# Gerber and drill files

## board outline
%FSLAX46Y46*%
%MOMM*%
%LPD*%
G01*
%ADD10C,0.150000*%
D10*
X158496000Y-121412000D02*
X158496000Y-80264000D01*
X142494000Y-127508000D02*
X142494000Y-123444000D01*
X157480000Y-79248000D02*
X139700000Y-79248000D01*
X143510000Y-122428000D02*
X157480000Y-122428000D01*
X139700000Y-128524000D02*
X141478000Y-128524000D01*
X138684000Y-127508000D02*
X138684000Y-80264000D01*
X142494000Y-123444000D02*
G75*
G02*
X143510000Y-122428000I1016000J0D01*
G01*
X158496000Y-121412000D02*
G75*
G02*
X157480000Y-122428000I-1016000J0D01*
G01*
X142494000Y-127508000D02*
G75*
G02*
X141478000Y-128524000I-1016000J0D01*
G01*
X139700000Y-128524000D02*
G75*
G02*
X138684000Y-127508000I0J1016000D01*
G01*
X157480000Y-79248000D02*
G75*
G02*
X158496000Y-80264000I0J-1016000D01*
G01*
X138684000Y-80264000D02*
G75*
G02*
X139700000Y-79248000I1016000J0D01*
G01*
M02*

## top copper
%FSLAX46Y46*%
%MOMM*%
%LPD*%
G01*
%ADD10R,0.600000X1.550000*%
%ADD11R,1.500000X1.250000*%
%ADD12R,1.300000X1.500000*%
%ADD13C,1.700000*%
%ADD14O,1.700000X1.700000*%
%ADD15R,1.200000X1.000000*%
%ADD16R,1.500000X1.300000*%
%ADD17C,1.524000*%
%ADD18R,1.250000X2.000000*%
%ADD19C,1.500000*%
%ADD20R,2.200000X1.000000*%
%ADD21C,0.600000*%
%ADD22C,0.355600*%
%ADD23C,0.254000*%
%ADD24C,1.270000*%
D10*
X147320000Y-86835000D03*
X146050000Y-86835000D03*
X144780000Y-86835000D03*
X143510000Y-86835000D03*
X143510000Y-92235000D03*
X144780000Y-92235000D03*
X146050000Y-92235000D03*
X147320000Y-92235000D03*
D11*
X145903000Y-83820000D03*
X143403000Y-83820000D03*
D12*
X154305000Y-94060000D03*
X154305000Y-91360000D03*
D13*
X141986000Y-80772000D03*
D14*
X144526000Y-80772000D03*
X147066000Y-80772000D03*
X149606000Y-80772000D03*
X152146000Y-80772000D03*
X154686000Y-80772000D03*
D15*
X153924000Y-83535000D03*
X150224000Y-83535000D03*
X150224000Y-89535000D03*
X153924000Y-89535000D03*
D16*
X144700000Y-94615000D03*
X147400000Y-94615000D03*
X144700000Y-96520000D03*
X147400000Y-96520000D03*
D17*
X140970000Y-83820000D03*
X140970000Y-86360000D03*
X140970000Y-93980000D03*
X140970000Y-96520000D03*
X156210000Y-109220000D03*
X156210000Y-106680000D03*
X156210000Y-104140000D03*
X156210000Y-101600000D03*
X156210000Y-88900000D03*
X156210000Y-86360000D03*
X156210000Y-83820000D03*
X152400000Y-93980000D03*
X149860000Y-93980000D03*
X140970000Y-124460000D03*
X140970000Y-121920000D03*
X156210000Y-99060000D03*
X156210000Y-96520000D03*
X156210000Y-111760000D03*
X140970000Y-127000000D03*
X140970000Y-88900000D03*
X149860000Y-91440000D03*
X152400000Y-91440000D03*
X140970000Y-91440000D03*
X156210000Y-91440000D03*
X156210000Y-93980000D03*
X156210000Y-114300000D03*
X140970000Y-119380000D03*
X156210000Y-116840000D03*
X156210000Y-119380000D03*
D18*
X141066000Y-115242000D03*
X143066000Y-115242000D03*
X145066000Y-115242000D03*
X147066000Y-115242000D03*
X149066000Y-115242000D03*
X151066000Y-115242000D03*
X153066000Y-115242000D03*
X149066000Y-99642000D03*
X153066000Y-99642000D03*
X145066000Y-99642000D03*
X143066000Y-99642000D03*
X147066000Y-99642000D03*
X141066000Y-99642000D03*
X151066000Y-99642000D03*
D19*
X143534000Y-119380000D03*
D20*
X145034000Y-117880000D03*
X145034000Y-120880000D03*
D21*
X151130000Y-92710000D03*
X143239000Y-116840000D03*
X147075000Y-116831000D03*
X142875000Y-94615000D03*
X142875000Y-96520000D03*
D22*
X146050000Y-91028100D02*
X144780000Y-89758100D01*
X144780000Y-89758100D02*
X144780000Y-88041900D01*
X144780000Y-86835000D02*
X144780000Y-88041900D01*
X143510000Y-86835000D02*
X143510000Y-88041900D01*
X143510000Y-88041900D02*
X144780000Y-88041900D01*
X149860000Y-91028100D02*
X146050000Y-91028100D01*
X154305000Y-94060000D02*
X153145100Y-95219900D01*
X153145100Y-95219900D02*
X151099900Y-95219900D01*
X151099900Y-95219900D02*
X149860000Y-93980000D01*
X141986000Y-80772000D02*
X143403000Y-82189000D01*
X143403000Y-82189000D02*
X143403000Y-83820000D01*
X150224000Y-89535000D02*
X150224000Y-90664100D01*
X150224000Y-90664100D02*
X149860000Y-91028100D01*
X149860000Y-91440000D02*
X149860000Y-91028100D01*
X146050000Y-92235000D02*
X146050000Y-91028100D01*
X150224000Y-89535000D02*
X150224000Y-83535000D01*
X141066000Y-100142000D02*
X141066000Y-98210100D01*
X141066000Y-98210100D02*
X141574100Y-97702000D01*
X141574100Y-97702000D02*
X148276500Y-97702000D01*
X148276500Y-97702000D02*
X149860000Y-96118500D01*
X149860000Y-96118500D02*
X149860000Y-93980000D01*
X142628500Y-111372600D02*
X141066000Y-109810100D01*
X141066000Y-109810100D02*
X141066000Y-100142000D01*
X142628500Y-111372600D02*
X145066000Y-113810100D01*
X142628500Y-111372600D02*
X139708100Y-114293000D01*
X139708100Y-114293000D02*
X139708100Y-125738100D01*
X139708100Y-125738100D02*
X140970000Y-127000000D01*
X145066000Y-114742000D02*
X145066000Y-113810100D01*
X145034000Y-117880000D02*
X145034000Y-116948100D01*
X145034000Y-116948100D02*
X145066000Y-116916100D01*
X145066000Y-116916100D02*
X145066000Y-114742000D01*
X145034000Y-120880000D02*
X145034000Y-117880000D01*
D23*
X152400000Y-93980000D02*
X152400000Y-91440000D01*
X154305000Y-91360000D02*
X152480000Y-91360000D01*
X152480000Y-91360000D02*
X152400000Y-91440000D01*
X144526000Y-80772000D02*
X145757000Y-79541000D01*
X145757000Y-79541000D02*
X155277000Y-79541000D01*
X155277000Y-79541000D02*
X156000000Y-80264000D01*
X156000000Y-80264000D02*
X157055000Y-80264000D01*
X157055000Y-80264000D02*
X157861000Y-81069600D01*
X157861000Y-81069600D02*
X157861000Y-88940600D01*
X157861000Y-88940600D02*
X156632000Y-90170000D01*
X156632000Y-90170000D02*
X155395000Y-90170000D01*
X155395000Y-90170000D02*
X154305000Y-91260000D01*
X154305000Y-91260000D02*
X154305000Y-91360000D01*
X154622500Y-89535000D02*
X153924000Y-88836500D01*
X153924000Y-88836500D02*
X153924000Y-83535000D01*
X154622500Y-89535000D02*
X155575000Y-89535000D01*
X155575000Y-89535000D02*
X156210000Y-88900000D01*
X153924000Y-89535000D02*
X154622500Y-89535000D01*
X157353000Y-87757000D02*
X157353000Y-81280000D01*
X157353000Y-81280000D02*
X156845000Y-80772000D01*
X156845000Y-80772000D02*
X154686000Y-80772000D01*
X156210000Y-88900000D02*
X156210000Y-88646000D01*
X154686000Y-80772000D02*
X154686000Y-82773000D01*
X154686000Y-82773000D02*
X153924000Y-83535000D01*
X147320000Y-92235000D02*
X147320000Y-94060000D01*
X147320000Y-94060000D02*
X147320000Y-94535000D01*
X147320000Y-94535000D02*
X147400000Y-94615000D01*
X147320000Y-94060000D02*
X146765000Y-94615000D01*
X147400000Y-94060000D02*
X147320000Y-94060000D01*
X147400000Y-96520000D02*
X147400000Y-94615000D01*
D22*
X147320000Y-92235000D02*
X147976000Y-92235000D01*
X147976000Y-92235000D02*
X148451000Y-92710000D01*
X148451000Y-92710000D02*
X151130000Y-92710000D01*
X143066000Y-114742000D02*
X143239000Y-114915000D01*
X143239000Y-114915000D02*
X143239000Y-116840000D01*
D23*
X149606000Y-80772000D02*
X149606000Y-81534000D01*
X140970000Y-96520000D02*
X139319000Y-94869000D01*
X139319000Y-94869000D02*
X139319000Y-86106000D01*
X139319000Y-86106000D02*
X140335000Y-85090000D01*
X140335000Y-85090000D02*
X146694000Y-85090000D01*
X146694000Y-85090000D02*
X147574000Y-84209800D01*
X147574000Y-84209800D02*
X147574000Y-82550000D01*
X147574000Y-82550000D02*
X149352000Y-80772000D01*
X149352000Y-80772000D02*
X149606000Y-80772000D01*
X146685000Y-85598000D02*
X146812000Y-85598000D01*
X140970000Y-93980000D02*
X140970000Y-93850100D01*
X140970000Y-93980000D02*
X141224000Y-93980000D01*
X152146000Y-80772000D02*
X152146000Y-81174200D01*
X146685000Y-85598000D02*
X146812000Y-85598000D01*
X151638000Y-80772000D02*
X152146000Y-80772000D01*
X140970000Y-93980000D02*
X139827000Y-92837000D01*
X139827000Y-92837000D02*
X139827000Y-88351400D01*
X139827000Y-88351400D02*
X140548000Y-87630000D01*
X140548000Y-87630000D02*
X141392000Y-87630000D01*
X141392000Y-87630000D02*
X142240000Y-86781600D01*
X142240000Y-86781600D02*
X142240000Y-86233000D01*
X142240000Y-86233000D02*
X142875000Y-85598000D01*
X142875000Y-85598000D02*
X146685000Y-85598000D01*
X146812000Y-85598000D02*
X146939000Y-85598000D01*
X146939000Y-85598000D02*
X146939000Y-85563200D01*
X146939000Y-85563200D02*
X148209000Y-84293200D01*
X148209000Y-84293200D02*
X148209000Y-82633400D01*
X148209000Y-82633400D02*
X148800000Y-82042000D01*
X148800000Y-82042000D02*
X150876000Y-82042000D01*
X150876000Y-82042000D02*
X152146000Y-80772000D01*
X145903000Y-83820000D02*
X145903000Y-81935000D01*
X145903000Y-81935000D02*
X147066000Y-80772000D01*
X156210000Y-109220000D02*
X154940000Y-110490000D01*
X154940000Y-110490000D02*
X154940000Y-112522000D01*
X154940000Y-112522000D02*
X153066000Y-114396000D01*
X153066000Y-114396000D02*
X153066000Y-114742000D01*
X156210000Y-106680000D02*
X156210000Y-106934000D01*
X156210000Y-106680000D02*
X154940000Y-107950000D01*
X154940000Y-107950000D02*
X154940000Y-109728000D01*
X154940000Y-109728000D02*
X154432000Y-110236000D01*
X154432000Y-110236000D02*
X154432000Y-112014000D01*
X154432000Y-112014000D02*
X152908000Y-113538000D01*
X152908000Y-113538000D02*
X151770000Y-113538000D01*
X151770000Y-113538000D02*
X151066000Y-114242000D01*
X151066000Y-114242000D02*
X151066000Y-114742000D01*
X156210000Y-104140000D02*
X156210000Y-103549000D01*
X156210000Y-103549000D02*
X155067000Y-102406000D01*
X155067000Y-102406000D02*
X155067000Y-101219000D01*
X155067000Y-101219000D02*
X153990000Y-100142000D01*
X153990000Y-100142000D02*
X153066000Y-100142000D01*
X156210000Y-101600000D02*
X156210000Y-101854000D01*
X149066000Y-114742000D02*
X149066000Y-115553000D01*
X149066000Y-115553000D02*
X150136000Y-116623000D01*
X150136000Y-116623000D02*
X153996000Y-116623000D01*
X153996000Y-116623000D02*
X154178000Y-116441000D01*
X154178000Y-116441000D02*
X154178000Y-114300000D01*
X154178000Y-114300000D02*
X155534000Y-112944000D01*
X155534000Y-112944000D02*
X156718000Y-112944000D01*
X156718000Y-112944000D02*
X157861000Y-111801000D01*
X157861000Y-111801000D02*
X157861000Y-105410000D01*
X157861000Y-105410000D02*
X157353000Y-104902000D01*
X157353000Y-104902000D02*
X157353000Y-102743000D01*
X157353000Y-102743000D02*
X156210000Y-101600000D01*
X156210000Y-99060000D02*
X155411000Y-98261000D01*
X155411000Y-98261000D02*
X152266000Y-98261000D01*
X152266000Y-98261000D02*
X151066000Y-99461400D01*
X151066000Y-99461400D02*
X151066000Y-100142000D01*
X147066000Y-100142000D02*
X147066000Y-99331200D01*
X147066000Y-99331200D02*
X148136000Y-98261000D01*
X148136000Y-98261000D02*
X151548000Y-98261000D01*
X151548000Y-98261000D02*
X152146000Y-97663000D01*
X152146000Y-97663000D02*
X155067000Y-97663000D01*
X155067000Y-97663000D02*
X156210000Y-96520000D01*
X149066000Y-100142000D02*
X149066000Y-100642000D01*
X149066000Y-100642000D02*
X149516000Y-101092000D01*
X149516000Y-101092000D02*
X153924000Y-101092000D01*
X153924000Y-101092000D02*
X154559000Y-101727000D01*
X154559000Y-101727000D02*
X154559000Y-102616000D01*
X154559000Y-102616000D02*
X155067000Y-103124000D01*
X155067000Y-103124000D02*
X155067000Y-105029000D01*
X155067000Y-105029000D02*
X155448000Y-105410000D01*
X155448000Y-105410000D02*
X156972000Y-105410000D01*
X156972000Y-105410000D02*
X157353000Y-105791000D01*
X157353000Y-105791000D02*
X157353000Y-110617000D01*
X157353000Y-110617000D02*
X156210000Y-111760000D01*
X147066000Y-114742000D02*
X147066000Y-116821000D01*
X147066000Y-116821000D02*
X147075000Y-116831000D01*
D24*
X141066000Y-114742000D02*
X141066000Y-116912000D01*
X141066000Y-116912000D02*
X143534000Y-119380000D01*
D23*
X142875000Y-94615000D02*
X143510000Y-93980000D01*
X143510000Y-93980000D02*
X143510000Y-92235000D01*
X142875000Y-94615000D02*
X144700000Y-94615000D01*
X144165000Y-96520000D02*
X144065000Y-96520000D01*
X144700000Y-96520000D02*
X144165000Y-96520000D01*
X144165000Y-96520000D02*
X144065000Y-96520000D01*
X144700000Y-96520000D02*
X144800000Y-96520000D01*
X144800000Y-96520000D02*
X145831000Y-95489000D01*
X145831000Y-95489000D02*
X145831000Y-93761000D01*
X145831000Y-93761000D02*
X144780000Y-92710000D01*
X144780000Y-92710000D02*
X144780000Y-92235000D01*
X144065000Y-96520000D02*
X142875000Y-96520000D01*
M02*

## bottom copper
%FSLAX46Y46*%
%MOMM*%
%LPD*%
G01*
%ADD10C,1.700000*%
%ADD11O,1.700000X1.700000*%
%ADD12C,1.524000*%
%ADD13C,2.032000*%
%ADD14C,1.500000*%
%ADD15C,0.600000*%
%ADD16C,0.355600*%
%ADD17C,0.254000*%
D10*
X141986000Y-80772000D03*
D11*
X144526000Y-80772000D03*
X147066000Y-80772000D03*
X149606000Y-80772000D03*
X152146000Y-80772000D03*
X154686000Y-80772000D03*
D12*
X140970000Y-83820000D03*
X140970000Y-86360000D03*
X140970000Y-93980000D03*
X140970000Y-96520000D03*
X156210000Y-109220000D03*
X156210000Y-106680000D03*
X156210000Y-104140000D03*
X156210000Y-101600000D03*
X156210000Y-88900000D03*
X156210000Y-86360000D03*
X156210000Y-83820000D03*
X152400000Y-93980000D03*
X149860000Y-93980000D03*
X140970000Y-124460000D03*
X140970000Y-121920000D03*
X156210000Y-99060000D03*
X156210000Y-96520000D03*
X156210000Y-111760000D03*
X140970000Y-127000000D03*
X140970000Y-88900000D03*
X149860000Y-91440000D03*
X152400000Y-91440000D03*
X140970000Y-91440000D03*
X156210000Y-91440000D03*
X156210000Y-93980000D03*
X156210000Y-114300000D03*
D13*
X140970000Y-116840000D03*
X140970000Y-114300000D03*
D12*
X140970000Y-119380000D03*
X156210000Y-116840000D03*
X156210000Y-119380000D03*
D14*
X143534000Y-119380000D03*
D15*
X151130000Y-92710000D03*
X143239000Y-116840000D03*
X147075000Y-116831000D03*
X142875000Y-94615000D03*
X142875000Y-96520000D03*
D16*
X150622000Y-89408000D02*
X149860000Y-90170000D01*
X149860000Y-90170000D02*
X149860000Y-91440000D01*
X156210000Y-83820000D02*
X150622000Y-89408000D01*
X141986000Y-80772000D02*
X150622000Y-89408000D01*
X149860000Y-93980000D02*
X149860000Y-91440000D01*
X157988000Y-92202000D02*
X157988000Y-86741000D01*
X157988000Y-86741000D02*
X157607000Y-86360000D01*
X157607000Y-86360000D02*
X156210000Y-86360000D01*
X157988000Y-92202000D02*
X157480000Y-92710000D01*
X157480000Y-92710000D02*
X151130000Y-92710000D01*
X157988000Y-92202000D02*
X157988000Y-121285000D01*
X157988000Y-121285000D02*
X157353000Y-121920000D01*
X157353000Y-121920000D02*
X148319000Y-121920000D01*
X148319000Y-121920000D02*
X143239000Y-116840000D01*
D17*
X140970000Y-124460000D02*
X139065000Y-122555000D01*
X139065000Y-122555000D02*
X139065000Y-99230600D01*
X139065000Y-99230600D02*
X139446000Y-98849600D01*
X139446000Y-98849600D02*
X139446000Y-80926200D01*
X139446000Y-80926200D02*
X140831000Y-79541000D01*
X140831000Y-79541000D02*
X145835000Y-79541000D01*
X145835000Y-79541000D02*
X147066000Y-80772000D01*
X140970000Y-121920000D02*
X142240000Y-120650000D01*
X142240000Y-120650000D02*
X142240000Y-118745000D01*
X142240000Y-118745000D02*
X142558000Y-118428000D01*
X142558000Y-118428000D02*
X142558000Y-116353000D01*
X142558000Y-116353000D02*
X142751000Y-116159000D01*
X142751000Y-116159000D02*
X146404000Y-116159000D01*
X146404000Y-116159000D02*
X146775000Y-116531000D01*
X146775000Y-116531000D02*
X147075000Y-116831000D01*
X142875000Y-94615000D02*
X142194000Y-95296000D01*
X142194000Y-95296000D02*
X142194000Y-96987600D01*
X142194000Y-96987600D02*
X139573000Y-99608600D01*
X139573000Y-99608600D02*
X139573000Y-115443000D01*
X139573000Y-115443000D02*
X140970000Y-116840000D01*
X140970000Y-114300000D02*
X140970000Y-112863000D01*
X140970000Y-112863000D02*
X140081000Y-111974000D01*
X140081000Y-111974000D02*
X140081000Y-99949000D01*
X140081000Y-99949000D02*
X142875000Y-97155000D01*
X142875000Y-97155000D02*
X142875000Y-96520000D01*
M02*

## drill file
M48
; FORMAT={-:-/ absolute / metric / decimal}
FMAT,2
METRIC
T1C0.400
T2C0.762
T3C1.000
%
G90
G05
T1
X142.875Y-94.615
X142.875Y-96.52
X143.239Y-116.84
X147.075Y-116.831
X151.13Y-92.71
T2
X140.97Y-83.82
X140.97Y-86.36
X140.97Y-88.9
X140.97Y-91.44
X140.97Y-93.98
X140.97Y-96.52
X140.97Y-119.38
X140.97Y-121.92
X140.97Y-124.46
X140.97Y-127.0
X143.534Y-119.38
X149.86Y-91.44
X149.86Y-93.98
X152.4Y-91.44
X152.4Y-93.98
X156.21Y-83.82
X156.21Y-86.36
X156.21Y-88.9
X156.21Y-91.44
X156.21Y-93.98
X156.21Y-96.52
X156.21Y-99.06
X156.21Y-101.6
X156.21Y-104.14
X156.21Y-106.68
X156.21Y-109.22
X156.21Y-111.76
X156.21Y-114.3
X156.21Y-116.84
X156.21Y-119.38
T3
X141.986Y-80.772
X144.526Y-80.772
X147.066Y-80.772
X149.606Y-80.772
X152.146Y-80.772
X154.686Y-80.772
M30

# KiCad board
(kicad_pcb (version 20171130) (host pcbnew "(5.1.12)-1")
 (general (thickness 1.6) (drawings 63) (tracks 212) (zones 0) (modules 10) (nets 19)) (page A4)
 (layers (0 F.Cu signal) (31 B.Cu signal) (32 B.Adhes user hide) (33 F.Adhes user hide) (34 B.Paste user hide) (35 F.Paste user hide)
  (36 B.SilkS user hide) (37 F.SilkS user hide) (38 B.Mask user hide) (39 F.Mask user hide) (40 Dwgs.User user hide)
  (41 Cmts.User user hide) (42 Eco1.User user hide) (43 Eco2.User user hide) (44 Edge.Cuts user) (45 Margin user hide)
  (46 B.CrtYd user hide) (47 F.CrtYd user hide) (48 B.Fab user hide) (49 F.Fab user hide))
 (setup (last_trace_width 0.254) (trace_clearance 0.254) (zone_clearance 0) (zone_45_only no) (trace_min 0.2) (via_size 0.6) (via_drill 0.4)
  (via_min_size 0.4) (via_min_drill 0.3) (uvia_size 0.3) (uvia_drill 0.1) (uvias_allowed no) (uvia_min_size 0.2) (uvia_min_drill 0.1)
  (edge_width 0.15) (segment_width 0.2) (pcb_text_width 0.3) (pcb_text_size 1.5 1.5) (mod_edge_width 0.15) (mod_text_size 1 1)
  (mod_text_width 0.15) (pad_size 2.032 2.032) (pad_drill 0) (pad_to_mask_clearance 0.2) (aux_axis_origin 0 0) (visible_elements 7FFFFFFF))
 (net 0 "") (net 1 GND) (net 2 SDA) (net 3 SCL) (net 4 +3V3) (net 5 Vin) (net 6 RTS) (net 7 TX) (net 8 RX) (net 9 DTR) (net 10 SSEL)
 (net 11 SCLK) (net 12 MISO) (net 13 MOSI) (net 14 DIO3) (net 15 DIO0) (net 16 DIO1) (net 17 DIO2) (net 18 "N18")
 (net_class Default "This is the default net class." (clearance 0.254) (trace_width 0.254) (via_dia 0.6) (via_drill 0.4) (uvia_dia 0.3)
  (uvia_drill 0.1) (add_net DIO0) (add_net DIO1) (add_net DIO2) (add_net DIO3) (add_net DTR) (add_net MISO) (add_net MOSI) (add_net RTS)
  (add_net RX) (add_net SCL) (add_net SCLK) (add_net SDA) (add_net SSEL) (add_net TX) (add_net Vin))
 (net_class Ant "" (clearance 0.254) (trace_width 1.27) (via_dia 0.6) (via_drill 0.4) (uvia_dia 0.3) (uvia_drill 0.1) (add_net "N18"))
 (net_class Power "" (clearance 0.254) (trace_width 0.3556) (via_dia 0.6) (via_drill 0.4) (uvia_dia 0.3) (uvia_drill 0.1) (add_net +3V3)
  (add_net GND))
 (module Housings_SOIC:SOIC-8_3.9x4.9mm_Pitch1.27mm (layer F.Cu) (at 145.415 89.535 270)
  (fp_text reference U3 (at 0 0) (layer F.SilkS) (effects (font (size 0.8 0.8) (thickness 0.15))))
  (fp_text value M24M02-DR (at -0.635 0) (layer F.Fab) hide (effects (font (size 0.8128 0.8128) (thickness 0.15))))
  (pad 1 smd rect (at -2.7 -1.905 270) (size 1.55 0.6) (layers F.Cu F.Paste F.Mask))
  (pad 2 smd rect (at -2.7 -0.635 270) (size 1.55 0.6) (layers F.Cu F.Paste F.Mask))
  (pad 3 smd rect (at -2.7 0.635 270) (size 1.55 0.6) (layers F.Cu F.Paste F.Mask) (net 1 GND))
  (pad 4 smd rect (at -2.7 1.905 270) (size 1.55 0.6) (layers F.Cu F.Paste F.Mask) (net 1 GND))
  (pad 5 smd rect (at 2.7 1.905 270) (size 1.55 0.6) (layers F.Cu F.Paste F.Mask) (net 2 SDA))
  (pad 6 smd rect (at 2.7 0.635 270) (size 1.55 0.6) (layers F.Cu F.Paste F.Mask) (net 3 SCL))
  (pad 7 smd rect (at 2.7 -0.635 270) (size 1.55 0.6) (layers F.Cu F.Paste F.Mask) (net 1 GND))
  (pad 8 smd rect (at 2.7 -1.905 270) (size 1.55 0.6) (layers F.Cu F.Paste F.Mask) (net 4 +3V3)))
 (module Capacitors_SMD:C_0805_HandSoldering (layer F.Cu) (at 144.653 83.82 180)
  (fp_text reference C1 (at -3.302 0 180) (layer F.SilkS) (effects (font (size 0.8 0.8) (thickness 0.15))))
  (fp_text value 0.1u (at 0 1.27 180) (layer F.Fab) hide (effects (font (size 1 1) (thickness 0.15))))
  (pad 1 smd rect (at -1.25 0 180) (size 1.5 1.25) (layers F.Cu F.Paste F.Mask) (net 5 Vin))
  (pad 2 smd rect (at 1.25 0 180) (size 1.5 1.25) (layers F.Cu F.Paste F.Mask) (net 1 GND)))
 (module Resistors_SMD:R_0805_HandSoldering (layer F.Cu) (at 154.305 92.71 90)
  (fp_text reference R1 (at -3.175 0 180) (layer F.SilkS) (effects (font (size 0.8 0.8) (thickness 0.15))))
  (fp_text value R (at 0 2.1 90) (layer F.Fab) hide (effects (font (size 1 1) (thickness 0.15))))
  (pad 1 smd rect (at -1.35 0 90) (size 1.5 1.3) (layers F.Cu F.Paste F.Mask) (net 1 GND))
  (pad 2 smd rect (at 1.35 0 90) (size 1.5 1.3) (layers F.Cu F.Paste F.Mask) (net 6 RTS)))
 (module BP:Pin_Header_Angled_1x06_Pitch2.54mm (layer F.Cu) (at 141.986 80.772 90)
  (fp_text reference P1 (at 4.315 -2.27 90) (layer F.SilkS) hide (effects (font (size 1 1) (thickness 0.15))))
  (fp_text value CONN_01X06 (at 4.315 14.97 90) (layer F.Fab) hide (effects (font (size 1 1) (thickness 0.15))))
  (pad 1 thru_hole circle (at 0 0 90) (size 1.7 1.7) (drill 1) (layers *.Cu *.Mask) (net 1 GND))
  (pad 2 thru_hole oval (at 0 2.54 90) (size 1.7 1.7) (drill 1) (layers *.Cu *.Mask) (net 6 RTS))
  (pad 3 thru_hole oval (at 0 5.08 90) (size 1.7 1.7) (drill 1) (layers *.Cu *.Mask) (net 5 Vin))
  (pad 4 thru_hole oval (at 0 7.62 90) (size 1.7 1.7) (drill 1) (layers *.Cu *.Mask) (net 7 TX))
  (pad 5 thru_hole oval (at 0 10.16 90) (size 1.7 1.7) (drill 1) (layers *.Cu *.Mask) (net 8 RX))
  (pad 6 thru_hole oval (at 0 12.7 90) (size 1.7 1.7) (drill 1) (layers *.Cu *.Mask) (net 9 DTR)))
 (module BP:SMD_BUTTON (layer F.Cu) (at 152.074 86.535 270)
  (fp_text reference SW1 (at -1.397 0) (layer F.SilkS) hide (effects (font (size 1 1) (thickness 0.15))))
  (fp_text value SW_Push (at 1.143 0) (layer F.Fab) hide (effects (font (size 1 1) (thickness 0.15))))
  (pad 1 smd rect (at -3 -1.85 270) (size 1 1.2) (layers F.Cu F.Paste F.Mask) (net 9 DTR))
  (pad 2 smd rect (at -3 1.85 270) (size 1 1.2) (layers F.Cu F.Paste F.Mask) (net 1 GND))
  (pad 2 smd rect (at 3 1.85 270) (size 1 1.2) (layers F.Cu F.Paste F.Mask) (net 1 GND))
  (pad 1 smd rect (at 3 -1.85 270) (size 1 1.2) (layers F.Cu F.Paste F.Mask) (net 9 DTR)))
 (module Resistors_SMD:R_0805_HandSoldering (layer F.Cu) (at 146.05 94.615)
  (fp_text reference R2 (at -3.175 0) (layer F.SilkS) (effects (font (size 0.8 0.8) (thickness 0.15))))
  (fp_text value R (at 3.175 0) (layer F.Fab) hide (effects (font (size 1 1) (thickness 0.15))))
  (pad 1 smd rect (at -1.35 0) (size 1.5 1.3) (layers F.Cu F.Paste F.Mask) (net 2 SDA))
  (pad 2 smd rect (at 1.35 0) (size 1.5 1.3) (layers F.Cu F.Paste F.Mask) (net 4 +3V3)))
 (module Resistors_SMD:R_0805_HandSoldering (layer F.Cu) (at 146.05 96.52)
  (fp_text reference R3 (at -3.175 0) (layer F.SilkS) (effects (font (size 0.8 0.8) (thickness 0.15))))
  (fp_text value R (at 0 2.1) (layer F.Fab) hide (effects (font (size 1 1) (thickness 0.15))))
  (pad 1 smd rect (at -1.35 0) (size 1.5 1.3) (layers F.Cu F.Paste F.Mask) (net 3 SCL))
  (pad 2 smd rect (at 1.35 0) (size 1.5 1.3) (layers F.Cu F.Paste F.Mask) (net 4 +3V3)))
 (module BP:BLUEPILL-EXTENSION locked (layer F.Cu) (at 148.59 105.41)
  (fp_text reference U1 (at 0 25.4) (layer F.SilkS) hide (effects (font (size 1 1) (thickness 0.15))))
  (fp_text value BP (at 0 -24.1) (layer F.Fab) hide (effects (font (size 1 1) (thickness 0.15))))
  (pad PB13 thru_hole circle (at -7.62 -21.59) (size 1.524 1.524) (drill 0.762) (layers *.Cu *.Mask))
  (pad PB14 thru_hole circle (at -7.62 -19.05) (size 1.524 1.524) (drill 0.762) (layers *.Cu *.Mask))
  (pad PA9 thru_hole circle (at -7.62 -11.43) (size 1.524 1.524) (drill 0.762) (layers *.Cu *.Mask) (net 8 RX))
  (pad PA10 thru_hole circle (at -7.62 -8.89) (size 1.524 1.524) (drill 0.762) (layers *.Cu *.Mask) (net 7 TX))
  (pad PA4 thru_hole circle (at 7.62 3.81) (size 1.524 1.524) (drill 0.762) (layers *.Cu *.Mask) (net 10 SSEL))
  (pad PA5 thru_hole circle (at 7.62 1.27) (size 1.524 1.524) (drill 0.762) (layers *.Cu *.Mask) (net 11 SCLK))
  (pad PA6 thru_hole circle (at 7.62 -1.27) (size 1.524 1.524) (drill 0.762) (layers *.Cu *.Mask) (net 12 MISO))
  (pad PA7 thru_hole circle (at 7.62 -3.81) (size 1.524 1.524) (drill 0.762) (layers *.Cu *.Mask) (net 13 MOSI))
  (pad NRST thru_hole circle (at 7.62 -16.51) (size 1.524 1.524) (drill 0.762) (layers *.Cu *.Mask) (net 9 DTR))
  (pad 3V3 thru_hole circle (at 7.62 -19.05) (size 1.524 1.524) (drill 0.762) (layers *.Cu *.Mask) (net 4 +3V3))
  (pad G thru_hole circle (at 7.62 -21.59) (size 1.524 1.524) (drill 0.762) (layers *.Cu *.Mask) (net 1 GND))
  (pad BOOT thru_hole circle (at 3.81 -11.43) (size 1.524 1.524) (drill 0.762) (layers *.Cu *.Mask) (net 6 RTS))
  (pad PB2 thru_hole circle (at 1.27 -11.43) (size 1.524 1.524) (drill 0.762) (layers *.Cu *.Mask) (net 1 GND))
  (pad 5V thru_hole circle (at -7.62 19.05) (size 1.524 1.524) (drill 0.762) (layers *.Cu *.Mask) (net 5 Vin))
  (pad PB9 thru_hole circle (at -7.62 16.51) (size 1.524 1.524) (drill 0.762) (layers *.Cu *.Mask) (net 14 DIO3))
  (pad PB0 thru_hole circle (at 7.62 -6.35) (size 1.524 1.524) (drill 0.762) (layers *.Cu *.Mask) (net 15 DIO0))
  (pad PB1 thru_hole circle (at 7.62 -8.89) (size 1.524 1.524) (drill 0.762) (layers *.Cu *.Mask) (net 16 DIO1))
  (pad PA3 thru_hole circle (at 7.62 6.35) (size 1.524 1.524) (drill 0.762) (layers *.Cu *.Mask) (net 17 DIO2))
  (pad G thru_hole circle (at -7.62 21.59) (size 1.524 1.524) (drill 0.762) (layers *.Cu *.Mask) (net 1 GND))
  (pad PB15 thru_hole circle (at -7.62 -16.51) (size 1.524 1.524) (drill 0.762) (layers *.Cu *.Mask))
  (pad PB2 thru_hole circle (at 1.27 -13.97) (size 1.524 1.524) (drill 0.762) (layers *.Cu *.Mask) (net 1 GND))
  (pad BOOT thru_hole circle (at 3.81 -13.97) (size 1.524 1.524) (drill 0.762) (layers *.Cu *.Mask) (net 6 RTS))
  (pad PA8 thru_hole circle (at -7.62 -13.97) (size 1.524 1.524) (drill 0.762) (layers *.Cu *.Mask))
  (pad PB11 thru_hole circle (at 7.62 -13.97) (size 1.524 1.524) (drill 0.762) (layers *.Cu *.Mask))
  (pad PB10 thru_hole circle (at 7.62 -11.43) (size 1.524 1.524) (drill 0.762) (layers *.Cu *.Mask))
  (pad PA2 thru_hole circle (at 7.62 8.89) (size 1.524 1.524) (drill 0.762) (layers *.Cu *.Mask))
  (pad PB7 smd circle (at -7.62 11.43) (size 2.032 2.032) (layers B.Cu B.Mask) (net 2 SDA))
  (pad PB6 smd circle (at -7.62 8.89) (size 2.032 2.032) (layers B.Cu B.Mask) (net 3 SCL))
  (pad PB8 thru_hole circle (at -7.62 13.97) (size 1.524 1.524) (drill 0.762) (layers *.Cu *.Mask))
  (pad PA1 thru_hole circle (at 7.62 11.43) (size 1.524 1.524) (drill 0.762) (layers *.Cu *.Mask))
  (pad PA0 thru_hole circle (at 7.62 13.97) (size 1.524 1.524) (drill 0.762) (layers *.Cu *.Mask)))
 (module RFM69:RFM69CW (layer F.Cu) (at 147.066 107.442 270)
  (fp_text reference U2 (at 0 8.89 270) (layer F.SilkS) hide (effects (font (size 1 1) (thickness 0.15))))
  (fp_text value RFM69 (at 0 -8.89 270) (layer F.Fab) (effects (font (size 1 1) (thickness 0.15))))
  (pad 1 smd rect (at 7.3 6 270) (size 2 1.25) (drill (offset 0.5 0)) (layers F.Cu F.Paste F.Mask) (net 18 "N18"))
  (pad 2 smd rect (at 7.3 4 270) (size 2 1.25) (drill (offset 0.5 0)) (layers F.Cu F.Paste F.Mask) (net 4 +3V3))
  (pad 3 smd rect (at 7.3 2 270) (size 2 1.25) (drill (offset 0.5 0)) (layers F.Cu F.Paste F.Mask) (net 1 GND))
  (pad 4 smd rect (at 7.3 0 270) (size 2 1.25) (drill (offset 0.5 0)) (layers F.Cu F.Paste F.Mask) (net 14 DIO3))
  (pad 5 smd rect (at 7.3 -2 270) (size 2 1.25) (drill (offset 0.5 0)) (layers F.Cu F.Paste F.Mask) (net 13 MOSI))
  (pad 6 smd rect (at 7.3 -4 270) (size 2 1.25) (drill (offset 0.5 0)) (layers F.Cu F.Paste F.Mask) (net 11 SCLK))
  (pad 7 smd rect (at 7.3 -6 270) (size 2 1.25) (drill (offset 0.5 0)) (layers F.Cu F.Paste F.Mask) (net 10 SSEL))
  (pad 10 smd rect (at -7.3 -2 270) (size 2 1.25) (drill (offset -0.5 0)) (layers F.Cu F.Paste F.Mask) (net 17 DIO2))
  (pad 8 smd rect (at -7.3 -6 270) (size 2 1.25) (drill (offset -0.5 0)) (layers F.Cu F.Paste F.Mask) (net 12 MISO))
  (pad 12 smd rect (at -7.3 2 270) (size 2 1.25) (drill (offset -0.5 0)) (layers F.Cu F.Paste F.Mask))
  (pad 13 smd rect (at -7.3 4 270) (size 2 1.25) (drill (offset -0.5 0)) (layers F.Cu F.Paste F.Mask))
  (pad 11 smd rect (at -7.3 0 270) (size 2 1.25) (drill (offset -0.5 0)) (layers F.Cu F.Paste F.Mask) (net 16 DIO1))
  (pad 14 smd rect (at -7.3 6 270) (size 2 1.25) (drill (offset -0.5 0)) (layers F.Cu F.Paste F.Mask) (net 1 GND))
  (pad 9 smd rect (at -7.3 -4 270) (size 2 1.25) (drill (offset -0.5 0)) (layers F.Cu F.Paste F.Mask) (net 15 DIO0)))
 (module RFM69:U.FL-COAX (layer F.Cu) (at 145.034 119.38)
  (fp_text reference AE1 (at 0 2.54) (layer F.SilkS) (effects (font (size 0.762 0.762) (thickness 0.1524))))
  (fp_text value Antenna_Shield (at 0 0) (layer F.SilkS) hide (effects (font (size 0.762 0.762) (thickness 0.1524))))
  (pad 1 thru_hole circle (at -1.5 0) (size 1.5 1.5) (drill 0.762) (layers *.Cu *.Mask) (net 18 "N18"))
  (pad 2 smd rect (at 0 -1.5) (size 2.2 1) (layers F.Cu F.Paste F.Mask) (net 1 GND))
  (pad 2 smd rect (at 0 1.5) (size 2.2 1) (layers F.Cu F.Paste F.Mask) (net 1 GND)))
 (gr_line (start 158.496 121.412) (end 158.496 80.264) (layer Edge.Cuts) (width 0.15))
 (gr_line (start 142.494 127.508) (end 142.494 123.444) (layer Edge.Cuts) (width 0.15))
 (gr_line (start 157.48 79.248) (end 139.7 79.248) (angle 90) (layer Edge.Cuts) (width 0.15))
 (gr_line (start 143.51 122.428) (end 157.48 122.428) (angle 90) (layer Edge.Cuts) (width 0.15))
 (gr_line (start 139.7 128.524) (end 141.478 128.524) (angle 90) (layer Edge.Cuts) (width 0.15))
 (gr_line (start 138.684 127.508) (end 138.684 80.264) (angle 90) (layer Edge.Cuts) (width 0.15))
 (gr_arc (start 143.51 123.444) (end 142.494 123.444) (angle 90) (layer Edge.Cuts) (width 0.15))
 (gr_arc (start 157.48 121.412) (end 158.496 121.412) (angle 90) (layer Edge.Cuts) (width 0.15))
 (gr_arc (start 141.478 127.508) (end 142.494 127.508) (angle 90) (layer Edge.Cuts) (width 0.15))
 (gr_arc (start 139.7 127.508) (end 139.7 128.524) (angle 90) (layer Edge.Cuts) (width 0.15))
 (gr_arc (start 157.48 80.264) (end 157.48 79.248) (angle 90) (layer Edge.Cuts) (width 0.15))
 (gr_arc (start 139.7 80.264) (end 138.684 80.264) (angle 90) (layer Edge.Cuts) (width 0.15))
 (segment (start 146.05 91.0281) (end 144.78 89.7581) (width 0.3556) (layer F.Cu) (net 1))
 (segment (start 144.78 89.7581) (end 144.78 88.0419) (width 0.3556) (layer F.Cu) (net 1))
 (segment (start 144.78 86.835) (end 144.78 88.0419) (width 0.3556) (layer F.Cu) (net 1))
 (segment (start 143.51 86.835) (end 143.51 88.0419) (width 0.3556) (layer F.Cu) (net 1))
 (segment (start 143.51 88.0419) (end 144.78 88.0419) (width 0.3556) (layer F.Cu) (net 1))
 (segment (start 149.86 91.0281) (end 146.05 91.0281) (width 0.3556) (layer F.Cu) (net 1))
 (segment (start 150.622 89.408) (end 149.86 90.17) (width 0.3556) (layer B.Cu) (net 1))
 (segment (start 149.86 90.17) (end 149.86 91.44) (width 0.3556) (layer B.Cu) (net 1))
 (segment (start 156.21 83.82) (end 150.622 89.408) (width 0.3556) (layer B.Cu) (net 1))
 (segment (start 141.986 80.772) (end 150.622 89.408) (width 0.3556) (layer B.Cu) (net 1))
 (segment (start 154.305 94.06) (end 153.1451 95.2199) (width 0.3556) (layer F.Cu) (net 1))
 (segment (start 153.1451 95.2199) (end 151.0999 95.2199) (width 0.3556) (layer F.Cu) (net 1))
 (segment (start 151.0999 95.2199) (end 149.86 93.98) (width 0.3556) (layer F.Cu) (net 1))
 (segment (start 141.986 80.772) (end 143.403 82.189) (width 0.3556) (layer F.Cu) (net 1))
 (segment (start 143.403 82.189) (end 143.403 83.82) (width 0.3556) (layer F.Cu) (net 1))
 (segment (start 150.224 89.535) (end 150.224 90.6641) (width 0.3556) (layer F.Cu) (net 1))
 (segment (start 150.224 90.6641) (end 149.86 91.0281) (width 0.3556) (layer F.Cu) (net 1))
 (segment (start 149.86 91.44) (end 149.86 91.0281) (width 0.3556) (layer F.Cu) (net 1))
 (segment (start 146.05 92.235) (end 146.05 91.0281) (width 0.3556) (layer F.Cu) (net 1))
 (segment (start 150.224 89.535) (end 150.224 83.535) (width 0.3556) (layer F.Cu) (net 1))
 (segment (start 149.86 93.98) (end 149.86 91.44) (width 0.3556) (layer B.Cu) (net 1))
 (segment (start 141.066 100.142) (end 141.066 98.2101) (width 0.3556) (layer F.Cu) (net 1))
 (segment (start 141.066 98.2101) (end 141.5741 97.702) (width 0.3556) (layer F.Cu) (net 1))
 (segment (start 141.5741 97.702) (end 148.2765 97.702) (width 0.3556) (layer F.Cu) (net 1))
 (segment (start 148.2765 97.702) (end 149.86 96.1185) (width 0.3556) (layer F.Cu) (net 1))
 (segment (start 149.86 96.1185) (end 149.86 93.98) (width 0.3556) (layer F.Cu) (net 1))
 (segment (start 142.6285 111.3726) (end 141.066 109.8101) (width 0.3556) (layer F.Cu) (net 1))
 (segment (start 141.066 109.8101) (end 141.066 100.142) (width 0.3556) (layer F.Cu) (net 1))
 (segment (start 142.6285 111.3726) (end 145.066 113.8101) (width 0.3556) (layer F.Cu) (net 1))
 (segment (start 142.6285 111.3726) (end 139.7081 114.293) (width 0.3556) (layer F.Cu) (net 1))
 (segment (start 139.7081 114.293) (end 139.7081 125.7381) (width 0.3556) (layer F.Cu) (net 1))
 (segment (start 139.7081 125.7381) (end 140.97 127) (width 0.3556) (layer F.Cu) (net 1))
 (segment (start 145.066 114.742) (end 145.066 113.8101) (width 0.3556) (layer F.Cu) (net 1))
 (segment (start 145.034 117.88) (end 145.034 116.9481) (width 0.3556) (layer F.Cu) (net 1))
 (segment (start 145.034 116.9481) (end 145.066 116.9161) (width 0.3556) (layer F.Cu) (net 1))
 (segment (start 145.066 116.9161) (end 145.066 114.742) (width 0.3556) (layer F.Cu) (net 1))
 (segment (start 145.034 120.88) (end 145.034 117.88) (width 0.3556) (layer F.Cu) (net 1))
 (segment (start 152.4 93.98) (end 152.4 91.44) (width 0.254) (layer F.Cu) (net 6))
 (segment (start 154.305 91.36) (end 152.48 91.36) (width 0.254) (layer F.Cu) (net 6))
 (segment (start 152.48 91.36) (end 152.4 91.44) (width 0.254) (layer F.Cu) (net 6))
 (segment (start 144.526 80.772) (end 145.757 79.541) (width 0.254) (layer F.Cu) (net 6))
 (segment (start 145.757 79.541) (end 155.277 79.541) (width 0.254) (layer F.Cu) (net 6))
 (segment (start 155.277 79.541) (end 156 80.264) (width 0.254) (layer F.Cu) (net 6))
 (segment (start 156 80.264) (end 157.055 80.264) (width 0.254) (layer F.Cu) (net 6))
 (segment (start 157.055 80.264) (end 157.861 81.0696) (width 0.254) (layer F.Cu) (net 6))
 (segment (start 157.861 81.0696) (end 157.861 88.9406) (width 0.254) (layer F.Cu) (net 6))
 (segment (start 157.861 88.9406) (end 156.632 90.17) (width 0.254) (layer F.Cu) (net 6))
 (segment (start 156.632 90.17) (end 155.395 90.17) (width 0.254) (layer F.Cu) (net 6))
 (segment (start 155.395 90.17) (end 154.305 91.26) (width 0.254) (layer F.Cu) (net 6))
 (segment (start 154.305 91.26) (end 154.305 91.36) (width 0.254) (layer F.Cu) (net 6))
 (segment (start 154.6225 89.535) (end 153.924 88.8365) (width 0.254) (layer F.Cu) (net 9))
 (segment (start 153.924 88.8365) (end 153.924 83.535) (width 0.254) (layer F.Cu) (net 9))
 (segment (start 154.6225 89.535) (end 155.575 89.535) (width 0.254) (layer F.Cu) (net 9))
 (segment (start 155.575 89.535) (end 156.21 88.9) (width 0.254) (layer F.Cu) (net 9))
 (segment (start 153.924 89.535) (end 154.6225 89.535) (width 0.254) (layer F.Cu) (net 9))
 (segment (start 157.353 87.757) (end 157.353 81.28) (width 0.254) (layer F.Cu) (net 9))
 (segment (start 157.353 81.28) (end 156.845 80.772) (width 0.254) (layer F.Cu) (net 9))
 (segment (start 156.845 80.772) (end 154.686 80.772) (width 0.254) (layer F.Cu) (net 9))
 (segment (start 156.21 88.9) (end 156.21 88.646) (width 0.254) (layer F.Cu) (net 9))
 (segment (start 154.686 80.772) (end 154.686 82.773) (width 0.254) (layer F.Cu) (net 9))
 (segment (start 154.686 82.773) (end 153.924 83.535) (width 0.254) (layer F.Cu) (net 9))
 (segment (start 147.32 92.235) (end 147.32 94.06) (width 0.254) (layer F.Cu) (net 4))
 (segment (start 147.32 94.06) (end 147.32 94.535) (width 0.254) (layer F.Cu) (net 4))
 (segment (start 147.32 94.535) (end 147.4 94.615) (width 0.254) (layer F.Cu) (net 4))
 (segment (start 147.32 94.06) (end 146.765 94.615) (width 0.254) (layer F.Cu) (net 4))
 (segment (start 147.4 94.06) (end 147.32 94.06) (width 0.254) (layer F.Cu) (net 4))
 (segment (start 147.4 96.52) (end 147.4 94.615) (width 0.254) (layer F.Cu) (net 4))
 (segment (start 157.988 92.202) (end 157.988 86.741) (width 0.3556) (layer B.Cu) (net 4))
 (segment (start 157.988 86.741) (end 157.607 86.36) (width 0.3556) (layer B.Cu) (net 4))
 (segment (start 157.607 86.36) (end 156.21 86.36) (width 0.3556) (layer B.Cu) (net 4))
 (segment (start 157.988 92.202) (end 157.48 92.71) (width 0.3556) (layer B.Cu) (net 4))
 (segment (start 157.48 92.71) (end 151.13 92.71) (width 0.3556) (layer B.Cu) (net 4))
 (segment (start 147.32 92.235) (end 147.976 92.235) (width 0.3556) (layer F.Cu) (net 4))
 (segment (start 147.976 92.235) (end 148.451 92.71) (width 0.3556) (layer F.Cu) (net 4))
 (segment (start 148.451 92.71) (end 151.13 92.71) (width 0.3556) (layer F.Cu) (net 4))
 (segment (start 143.066 114.742) (end 143.239 114.915) (width 0.3556) (layer F.Cu) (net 4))
 (segment (start 143.239 114.915) (end 143.239 116.84) (width 0.3556) (layer F.Cu) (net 4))
 (segment (start 157.988 92.202) (end 157.988 121.285) (width 0.3556) (layer B.Cu) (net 4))
 (segment (start 157.988 121.285) (end 157.353 121.92) (width 0.3556) (layer B.Cu) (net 4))
 (segment (start 157.353 121.92) (end 148.319 121.92) (width 0.3556) (layer B.Cu) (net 4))
 (segment (start 148.319 121.92) (end 143.239 116.84) (width 0.3556) (layer B.Cu) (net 4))
 (via (at 151.13 92.71) (size 0.6) (layers F.Cu B.Cu) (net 4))
 (via (at 143.239 116.84) (size 0.6) (layers F.Cu B.Cu) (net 4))
 (segment (start 149.606 80.772) (end 149.606 81.534) (width 0.254) (layer F.Cu) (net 7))
 (segment (start 140.97 96.52) (end 139.319 94.869) (width 0.254) (layer F.Cu) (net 7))
 (segment (start 139.319 94.869) (end 139.319 86.106) (width 0.254) (layer F.Cu) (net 7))
 (segment (start 139.319 86.106) (end 140.335 85.09) (width 0.254) (layer F.Cu) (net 7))
 (segment (start 140.335 85.09) (end 146.694 85.09) (width 0.254) (layer F.Cu) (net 7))
 (segment (start 146.694 85.09) (end 147.574 84.2098) (width 0.254) (layer F.Cu) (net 7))
 (segment (start 147.574 84.2098) (end 147.574 82.55) (width 0.254) (layer F.Cu) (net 7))
 (segment (start 147.574 82.55) (end 149.352 80.772) (width 0.254) (layer F.Cu) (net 7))
 (segment (start 149.352 80.772) (end 149.606 80.772) (width 0.254) (layer F.Cu) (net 7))
 (segment (start 146.685 85.598) (end 146.812 85.598) (width 0.254) (layer F.Cu) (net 8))
 (segment (start 140.97 93.98) (end 140.97 93.8501) (width 0.254) (layer F.Cu) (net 8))
 (segment (start 140.97 93.98) (end 141.224 93.98) (width 0.254) (layer F.Cu) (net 8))
 (segment (start 152.146 80.772) (end 152.146 81.1742) (width 0.254) (layer F.Cu) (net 8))
 (segment (start 146.685 85.598) (end 146.812 85.598) (width 0.254) (layer F.Cu) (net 8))
 (segment (start 151.638 80.772) (end 152.146 80.772) (width 0.254) (layer F.Cu) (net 8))
 (segment (start 140.97 93.98) (end 139.827 92.837) (width 0.254) (layer F.Cu) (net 8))
 (segment (start 139.827 92.837) (end 139.827 88.3514) (width 0.254) (layer F.Cu) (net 8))
 (segment (start 139.827 88.3514) (end 140.548 87.63) (width 0.254) (layer F.Cu) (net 8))
 (segment (start 140.548 87.63) (end 141.392 87.63) (width 0.254) (layer F.Cu) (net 8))
 (segment (start 141.392 87.63) (end 142.24 86.7816) (width 0.254) (layer F.Cu) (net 8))
 (segment (start 142.24 86.7816) (end 142.24 86.233) (width 0.254) (layer F.Cu) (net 8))
 (segment (start 142.24 86.233) (end 142.875 85.598) (width 0.254) (layer F.Cu) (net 8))
 (segment (start 142.875 85.598) (end 146.685 85.598) (width 0.254) (layer F.Cu) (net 8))
 (segment (start 146.812 85.598) (end 146.939 85.598) (width 0.254) (layer F.Cu) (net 8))
 (segment (start 146.939 85.598) (end 146.939 85.5632) (width 0.254) (layer F.Cu) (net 8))
 (segment (start 146.939 85.5632) (end 148.209 84.2932) (width 0.254) (layer F.Cu) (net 8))
 (segment (start 148.209 84.2932) (end 148.209 82.6334) (width 0.254) (layer F.Cu) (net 8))
 (segment (start 148.209 82.6334) (end 148.8 82.042) (width 0.254) (layer F.Cu) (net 8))
 (segment (start 148.8 82.042) (end 150.876 82.042) (width 0.254) (layer F.Cu) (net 8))
 (segment (start 150.876 82.042) (end 152.146 80.772) (width 0.254) (layer F.Cu) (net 8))
 (segment (start 140.97 124.46) (end 139.065 122.555) (width 0.254) (layer B.Cu) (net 5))
 (segment (start 139.065 122.555) (end 139.065 99.2306) (width 0.254) (layer B.Cu) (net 5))
 (segment (start 139.065 99.2306) (end 139.446 98.8496) (width 0.254) (layer B.Cu) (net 5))
 (segment (start 139.446 98.8496) (end 139.446 80.9262) (width 0.254) (layer B.Cu) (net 5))
 (segment (start 139.446 80.9262) (end 140.831 79.541) (width 0.254) (layer B.Cu) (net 5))
 (segment (start 140.831 79.541) (end 145.835 79.541) (width 0.254) (layer B.Cu) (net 5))
 (segment (start 145.835 79.541) (end 147.066 80.772) (width 0.254) (layer B.Cu) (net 5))
 (segment (start 145.903 83.82) (end 145.903 81.935) (width 0.254) (layer F.Cu) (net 5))
 (segment (start 145.903 81.935) (end 147.066 80.772) (width 0.254) (layer F.Cu) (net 5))
 (segment (start 156.21 109.22) (end 154.94 110.49) (width 0.254) (layer F.Cu) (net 10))
 (segment (start 154.94 110.49) (end 154.94 112.522) (width 0.254) (layer F.Cu) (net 10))
 (segment (start 154.94 112.522) (end 153.066 114.396) (width 0.254) (layer F.Cu) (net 10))
 (segment (start 153.066 114.396) (end 153.066 114.742) (width 0.254) (layer F.Cu) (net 10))
 (segment (start 156.21 106.68) (end 156.21 106.934) (width 0.254) (layer F.Cu) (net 11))
 (segment (start 156.21 106.68) (end 154.94 107.95) (width 0.254) (layer F.Cu) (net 11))
 (segment (start 154.94 107.95) (end 154.94 109.728) (width 0.254) (layer F.Cu) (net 11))
 (segment (start 154.94 109.728) (end 154.432 110.236) (width 0.254) (layer F.Cu) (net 11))
 (segment (start 154.432 110.236) (end 154.432 112.014) (width 0.254) (layer F.Cu) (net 11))
 (segment (start 154.432 112.014) (end 152.908 113.538) (width 0.254) (layer F.Cu) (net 11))
 (segment (start 152.908 113.538) (end 151.77 113.538) (width 0.254) (layer F.Cu) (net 11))
 (segment (start 151.77 113.538) (end 151.066 114.242) (width 0.254) (layer F.Cu) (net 11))
 (segment (start 151.066 114.242) (end 151.066 114.742) (width 0.254) (layer F.Cu) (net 11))
 (segment (start 156.21 104.14) (end 156.21 103.549) (width 0.254) (layer F.Cu) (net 12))
 (segment (start 156.21 103.549) (end 155.067 102.406) (width 0.254) (layer F.Cu) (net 12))
 (segment (start 155.067 102.406) (end 155.067 101.219) (width 0.254) (layer F.Cu) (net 12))
 (segment (start 155.067 101.219) (end 153.99 100.142) (width 0.254) (layer F.Cu) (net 12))
 (segment (start 153.99 100.142) (end 153.066 100.142) (width 0.254) (layer F.Cu) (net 12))
 (segment (start 156.21 101.6) (end 156.21 101.854) (width 0.254) (layer F.Cu) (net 13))
 (segment (start 149.066 114.742) (end 149.066 115.553) (width 0.254) (layer F.Cu) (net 13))
 (segment (start 149.066 115.553) (end 150.136 116.623) (width 0.254) (layer F.Cu) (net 13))
 (segment (start 150.136 116.623) (end 153.996 116.623) (width 0.254) (layer F.Cu) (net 13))
 (segment (start 153.996 116.623) (end 154.178 116.441) (width 0.254) (layer F.Cu) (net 13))
 (segment (start 154.178 116.441) (end 154.178 114.3) (width 0.254) (layer F.Cu) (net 13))
 (segment (start 154.178 114.3) (end 155.534 112.944) (width 0.254) (layer F.Cu) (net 13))
 (segment (start 155.534 112.944) (end 156.718 112.944) (width 0.254) (layer F.Cu) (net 13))
 (segment (start 156.718 112.944) (end 157.861 111.801) (width 0.254) (layer F.Cu) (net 13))
 (segment (start 157.861 111.801) (end 157.861 105.41) (width 0.254) (layer F.Cu) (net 13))
 (segment (start 157.861 105.41) (end 157.353 104.902) (width 0.254) (layer F.Cu) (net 13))
 (segment (start 157.353 104.902) (end 157.353 102.743) (width 0.254) (layer F.Cu) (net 13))
 (segment (start 157.353 102.743) (end 156.21 101.6) (width 0.254) (layer F.Cu) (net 13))
 (segment (start 156.21 99.06) (end 155.411 98.261) (width 0.254) (layer F.Cu) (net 15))
 (segment (start 155.411 98.261) (end 152.266 98.261) (width 0.254) (layer F.Cu) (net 15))
 (segment (start 152.266 98.261) (end 151.066 99.4614) (width 0.254) (layer F.Cu) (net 15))
 (segment (start 151.066 99.4614) (end 151.066 100.142) (width 0.254) (layer F.Cu) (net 15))
 (segment (start 147.066 100.142) (end 147.066 99.3312) (width 0.254) (layer F.Cu) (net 16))
 (segment (start 147.066 99.3312) (end 148.136 98.261) (width 0.254) (layer F.Cu) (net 16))
 (segment (start 148.136 98.261) (end 151.548 98.261) (width 0.254) (layer F.Cu) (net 16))
 (segment (start 151.548 98.261) (end 152.146 97.663) (width 0.254) (layer F.Cu) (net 16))
 (segment (start 152.146 97.663) (end 155.067 97.663) (width 0.254) (layer F.Cu) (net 16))
 (segment (start 155.067 97.663) (end 156.21 96.52) (width 0.254) (layer F.Cu) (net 16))
 (segment (start 149.066 100.142) (end 149.066 100.642) (width 0.254) (layer F.Cu) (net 17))
 (segment (start 149.066 100.642) (end 149.516 101.092) (width 0.254) (layer F.Cu) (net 17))
 (segment (start 149.516 101.092) (end 153.924 101.092) (width 0.254) (layer F.Cu) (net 17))
 (segment (start 153.924 101.092) (end 154.559 101.727) (width 0.254) (layer F.Cu) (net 17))
 (segment (start 154.559 101.727) (end 154.559 102.616) (width 0.254) (layer F.Cu) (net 17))
 (segment (start 154.559 102.616) (end 155.067 103.124) (width 0.254) (layer F.Cu) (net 17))
 (segment (start 155.067 103.124) (end 155.067 105.029) (width 0.254) (layer F.Cu) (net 17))
 (segment (start 155.067 105.029) (end 155.448 105.41) (width 0.254) (layer F.Cu) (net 17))
 (segment (start 155.448 105.41) (end 156.972 105.41) (width 0.254) (layer F.Cu) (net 17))
 (segment (start 156.972 105.41) (end 157.353 105.791) (width 0.254) (layer F.Cu) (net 17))
 (segment (start 157.353 105.791) (end 157.353 110.617) (width 0.254) (layer F.Cu) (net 17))
 (segment (start 157.353 110.617) (end 156.21 111.76) (width 0.254) (layer F.Cu) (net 17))
 (segment (start 140.97 121.92) (end 142.24 120.65) (width 0.254) (layer B.Cu) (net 14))
 (segment (start 142.24 120.65) (end 142.24 118.745) (width 0.254) (layer B.Cu) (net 14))
 (segment (start 142.24 118.745) (end 142.558 118.428) (width 0.254) (layer B.Cu) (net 14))
 (segment (start 142.558 118.428) (end 142.558 116.353) (width 0.254) (layer B.Cu) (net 14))
 (segment (start 142.558 116.353) (end 142.751 116.159) (width 0.254) (layer B.Cu) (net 14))
 (segment (start 142.751 116.159) (end 146.404 116.159) (width 0.254) (layer B.Cu) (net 14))
 (segment (start 146.404 116.159) (end 146.775 116.531) (width 0.254) (layer B.Cu) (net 14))
 (segment (start 146.775 116.531) (end 147.075 116.831) (width 0.254) (layer B.Cu) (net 14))
 (segment (start 147.066 114.742) (end 147.066 116.821) (width 0.254) (layer F.Cu) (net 14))
 (segment (start 147.066 116.821) (end 147.075 116.831) (width 0.254) (layer F.Cu) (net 14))
 (via (at 147.075 116.831) (size 0.6) (layers F.Cu B.Cu) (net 14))
 (segment (start 141.066 114.742) (end 141.066 116.912) (width 1.27) (layer F.Cu) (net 18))
 (segment (start 141.066 116.912) (end 143.534 119.38) (width 1.27) (layer F.Cu) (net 18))
 (segment (start 142.875 94.615) (end 143.51 93.98) (width 0.254) (layer F.Cu) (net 2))
 (segment (start 143.51 93.98) (end 143.51 92.235) (width 0.254) (layer F.Cu) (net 2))
 (segment (start 142.875 94.615) (end 144.7 94.615) (width 0.254) (layer F.Cu) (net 2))
 (segment (start 142.875 94.615) (end 142.194 95.296) (width 0.254) (layer B.Cu) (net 2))
 (segment (start 142.194 95.296) (end 142.194 96.9876) (width 0.254) (layer B.Cu) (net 2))
 (segment (start 142.194 96.9876) (end 139.573 99.6086) (width 0.254) (layer B.Cu) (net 2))
 (segment (start 139.573 99.6086) (end 139.573 115.443) (width 0.254) (layer B.Cu) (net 2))
 (segment (start 139.573 115.443) (end 140.97 116.84) (width 0.254) (layer B.Cu) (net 2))
 (via (at 142.875 94.615) (size 0.6) (layers F.Cu B.Cu) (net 2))
 (segment (start 144.165 96.52) (end 144.065 96.52) (width 0.254) (layer F.Cu) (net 3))
 (segment (start 144.7 96.52) (end 144.165 96.52) (width 0.254) (layer F.Cu) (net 3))
 (segment (start 144.165 96.52) (end 144.065 96.52) (width 0.254) (layer F.Cu) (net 3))
 (segment (start 144.7 96.52) (end 144.8 96.52) (width 0.254) (layer F.Cu) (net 3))
 (segment (start 144.8 96.52) (end 145.831 95.489) (width 0.254) (layer F.Cu) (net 3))
 (segment (start 145.831 95.489) (end 145.831 93.761) (width 0.254) (layer F.Cu) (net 3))
 (segment (start 145.831 93.761) (end 144.78 92.71) (width 0.254) (layer F.Cu) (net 3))
 (segment (start 144.78 92.71) (end 144.78 92.235) (width 0.254) (layer F.Cu) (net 3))
 (segment (start 140.97 114.3) (end 140.97 112.863) (width 0.254) (layer B.Cu) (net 3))
 (segment (start 140.97 112.863) (end 140.081 111.974) (width 0.254) (layer B.Cu) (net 3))
 (segment (start 140.081 111.974) (end 140.081 99.949) (width 0.254) (layer B.Cu) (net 3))
 (segment (start 140.081 99.949) (end 142.875 97.155) (width 0.254) (layer B.Cu) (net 3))
 (segment (start 142.875 97.155) (end 142.875 96.52) (width 0.254) (layer B.Cu) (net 3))
 (segment (start 144.065 96.52) (end 142.875 96.52) (width 0.254) (layer F.Cu) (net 3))
 (via (at 142.875 96.52) (size 0.6) (layers F.Cu B.Cu) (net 3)))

